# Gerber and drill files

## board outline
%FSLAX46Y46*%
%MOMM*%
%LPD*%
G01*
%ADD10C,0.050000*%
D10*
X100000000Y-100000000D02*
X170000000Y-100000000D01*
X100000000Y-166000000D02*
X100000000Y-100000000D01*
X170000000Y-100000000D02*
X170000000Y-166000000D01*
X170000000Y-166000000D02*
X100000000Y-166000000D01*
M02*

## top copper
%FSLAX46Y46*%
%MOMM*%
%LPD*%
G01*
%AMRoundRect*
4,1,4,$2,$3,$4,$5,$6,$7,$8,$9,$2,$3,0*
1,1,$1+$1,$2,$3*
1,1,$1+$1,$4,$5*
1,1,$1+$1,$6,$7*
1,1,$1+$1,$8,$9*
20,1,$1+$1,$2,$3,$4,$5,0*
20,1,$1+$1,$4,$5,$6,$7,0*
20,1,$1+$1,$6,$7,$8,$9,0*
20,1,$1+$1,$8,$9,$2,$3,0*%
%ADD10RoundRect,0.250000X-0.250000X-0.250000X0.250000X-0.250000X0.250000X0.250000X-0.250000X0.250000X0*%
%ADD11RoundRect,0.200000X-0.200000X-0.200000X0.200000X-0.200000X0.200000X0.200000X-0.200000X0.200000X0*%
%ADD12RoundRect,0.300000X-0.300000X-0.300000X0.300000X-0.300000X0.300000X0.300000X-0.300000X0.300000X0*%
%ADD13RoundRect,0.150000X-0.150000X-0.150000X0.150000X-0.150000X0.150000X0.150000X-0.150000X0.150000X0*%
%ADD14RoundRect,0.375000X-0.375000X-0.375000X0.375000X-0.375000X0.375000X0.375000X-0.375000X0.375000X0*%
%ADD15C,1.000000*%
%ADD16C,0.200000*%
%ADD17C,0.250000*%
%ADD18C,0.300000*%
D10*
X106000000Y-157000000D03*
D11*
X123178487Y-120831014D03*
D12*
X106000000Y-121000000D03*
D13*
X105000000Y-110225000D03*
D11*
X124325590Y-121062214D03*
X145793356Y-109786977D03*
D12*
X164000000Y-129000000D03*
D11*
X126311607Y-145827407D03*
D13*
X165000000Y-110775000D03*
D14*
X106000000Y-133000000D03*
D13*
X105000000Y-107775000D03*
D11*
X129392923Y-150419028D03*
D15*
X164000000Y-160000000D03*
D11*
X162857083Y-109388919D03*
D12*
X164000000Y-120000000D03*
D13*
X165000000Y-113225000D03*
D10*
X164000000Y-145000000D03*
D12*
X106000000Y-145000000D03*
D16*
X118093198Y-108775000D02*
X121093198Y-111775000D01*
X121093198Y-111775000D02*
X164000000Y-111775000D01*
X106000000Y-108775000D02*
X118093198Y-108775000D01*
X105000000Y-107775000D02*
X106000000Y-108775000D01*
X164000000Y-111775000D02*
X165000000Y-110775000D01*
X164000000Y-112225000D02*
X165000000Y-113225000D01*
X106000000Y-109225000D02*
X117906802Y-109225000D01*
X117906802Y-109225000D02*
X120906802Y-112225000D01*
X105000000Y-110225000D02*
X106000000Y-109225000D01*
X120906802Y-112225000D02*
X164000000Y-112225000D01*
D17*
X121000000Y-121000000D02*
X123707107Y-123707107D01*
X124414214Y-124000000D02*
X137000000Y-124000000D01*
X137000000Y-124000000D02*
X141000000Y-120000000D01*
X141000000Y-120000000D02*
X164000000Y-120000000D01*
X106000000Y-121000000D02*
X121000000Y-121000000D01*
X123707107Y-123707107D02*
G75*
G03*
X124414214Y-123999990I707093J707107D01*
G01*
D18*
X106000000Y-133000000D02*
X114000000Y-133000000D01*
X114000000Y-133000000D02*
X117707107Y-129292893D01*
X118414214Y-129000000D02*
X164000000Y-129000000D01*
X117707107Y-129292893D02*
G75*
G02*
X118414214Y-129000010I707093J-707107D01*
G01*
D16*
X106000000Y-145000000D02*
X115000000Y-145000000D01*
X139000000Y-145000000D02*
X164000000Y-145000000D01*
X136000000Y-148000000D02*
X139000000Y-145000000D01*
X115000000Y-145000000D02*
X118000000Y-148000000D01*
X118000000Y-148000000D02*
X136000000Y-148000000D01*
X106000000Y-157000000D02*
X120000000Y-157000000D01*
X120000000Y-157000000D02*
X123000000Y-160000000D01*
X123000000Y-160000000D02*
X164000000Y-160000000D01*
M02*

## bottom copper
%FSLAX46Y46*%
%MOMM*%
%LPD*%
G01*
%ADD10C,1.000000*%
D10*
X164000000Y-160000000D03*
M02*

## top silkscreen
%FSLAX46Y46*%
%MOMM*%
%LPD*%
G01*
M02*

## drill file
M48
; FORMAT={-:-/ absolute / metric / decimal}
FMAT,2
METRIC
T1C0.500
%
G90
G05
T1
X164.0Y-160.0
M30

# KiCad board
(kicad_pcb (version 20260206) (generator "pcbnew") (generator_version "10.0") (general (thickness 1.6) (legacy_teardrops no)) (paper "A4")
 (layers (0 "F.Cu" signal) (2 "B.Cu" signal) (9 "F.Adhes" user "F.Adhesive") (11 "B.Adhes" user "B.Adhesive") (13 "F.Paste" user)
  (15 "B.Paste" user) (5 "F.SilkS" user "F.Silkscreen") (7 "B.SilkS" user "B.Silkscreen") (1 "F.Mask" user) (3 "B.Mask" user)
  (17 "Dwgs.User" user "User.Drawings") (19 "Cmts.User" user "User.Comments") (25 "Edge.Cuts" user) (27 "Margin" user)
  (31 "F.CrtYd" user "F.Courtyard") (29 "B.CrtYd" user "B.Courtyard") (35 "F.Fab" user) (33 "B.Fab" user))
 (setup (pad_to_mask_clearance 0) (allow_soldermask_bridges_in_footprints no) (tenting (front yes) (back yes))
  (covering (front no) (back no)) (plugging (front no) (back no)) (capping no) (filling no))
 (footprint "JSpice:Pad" (layer "F.Cu") (at 106 157)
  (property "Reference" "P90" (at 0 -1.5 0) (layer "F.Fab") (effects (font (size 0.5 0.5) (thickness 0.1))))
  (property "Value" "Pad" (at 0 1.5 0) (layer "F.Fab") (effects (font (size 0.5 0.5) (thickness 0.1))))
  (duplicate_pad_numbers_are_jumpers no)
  (pad "1" smd roundrect (at 0 0) (size 1 1) (layers "F.Cu" "F.Mask") (roundrect_rratio 0.25) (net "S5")))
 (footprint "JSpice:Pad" (layer "F.Cu") (at 123.178487 120.831014)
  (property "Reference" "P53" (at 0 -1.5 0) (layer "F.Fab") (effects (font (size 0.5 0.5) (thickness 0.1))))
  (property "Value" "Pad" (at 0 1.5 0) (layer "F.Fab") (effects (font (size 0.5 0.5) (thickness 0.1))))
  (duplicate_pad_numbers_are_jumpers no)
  (pad "1" smd roundrect (at 0 0) (size 0.8 0.8) (layers "F.Cu" "F.Mask") (roundrect_rratio 0.25) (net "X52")))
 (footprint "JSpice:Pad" (layer "F.Cu") (at 106 121)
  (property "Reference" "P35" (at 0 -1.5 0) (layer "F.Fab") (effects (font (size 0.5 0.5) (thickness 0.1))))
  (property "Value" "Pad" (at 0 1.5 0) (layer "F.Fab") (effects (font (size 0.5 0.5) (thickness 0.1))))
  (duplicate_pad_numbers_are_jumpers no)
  (pad "1" smd roundrect (at 0 0) (size 1.2 1.2) (layers "F.Cu" "F.Mask") (roundrect_rratio 0.25) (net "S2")))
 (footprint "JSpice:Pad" (layer "F.Cu") (at 105 110.225)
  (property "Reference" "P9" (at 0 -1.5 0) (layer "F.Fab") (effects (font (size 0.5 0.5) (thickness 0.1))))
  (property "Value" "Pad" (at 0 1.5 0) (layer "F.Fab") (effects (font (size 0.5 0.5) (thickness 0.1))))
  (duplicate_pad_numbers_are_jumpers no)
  (pad "1" smd roundrect (at 0 0) (size 0.6 0.6) (layers "F.Cu" "F.Mask") (roundrect_rratio 0.25) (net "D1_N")))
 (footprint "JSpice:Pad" (layer "F.Cu") (at 124.32559 121.062214)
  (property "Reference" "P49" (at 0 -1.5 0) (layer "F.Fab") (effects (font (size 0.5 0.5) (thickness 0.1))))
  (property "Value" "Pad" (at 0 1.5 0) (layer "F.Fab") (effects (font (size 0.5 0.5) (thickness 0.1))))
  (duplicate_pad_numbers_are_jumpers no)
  (pad "1" smd roundrect (at 0 0) (size 0.8 0.8) (layers "F.Cu" "F.Mask") (roundrect_rratio 0.25) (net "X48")))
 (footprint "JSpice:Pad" (layer "F.Cu") (at 145.793356 109.786977)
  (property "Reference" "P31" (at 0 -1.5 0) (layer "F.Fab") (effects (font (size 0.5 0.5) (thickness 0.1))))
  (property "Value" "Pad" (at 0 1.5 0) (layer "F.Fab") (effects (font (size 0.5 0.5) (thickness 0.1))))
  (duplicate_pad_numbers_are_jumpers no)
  (pad "1" smd roundrect (at 0 0) (size 0.8 0.8) (layers "F.Cu" "F.Mask") (roundrect_rratio 0.25) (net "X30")))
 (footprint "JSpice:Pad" (layer "F.Cu") (at 164 129)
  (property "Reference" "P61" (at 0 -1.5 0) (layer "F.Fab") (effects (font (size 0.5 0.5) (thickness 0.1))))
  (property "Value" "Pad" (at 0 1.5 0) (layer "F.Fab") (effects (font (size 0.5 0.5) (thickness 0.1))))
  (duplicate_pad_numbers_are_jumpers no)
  (pad "1" smd roundrect (at 0 0) (size 1.2 1.2) (layers "F.Cu" "F.Mask") (roundrect_rratio 0.25) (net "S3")))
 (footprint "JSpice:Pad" (layer "F.Cu") (at 126.311607 145.827407)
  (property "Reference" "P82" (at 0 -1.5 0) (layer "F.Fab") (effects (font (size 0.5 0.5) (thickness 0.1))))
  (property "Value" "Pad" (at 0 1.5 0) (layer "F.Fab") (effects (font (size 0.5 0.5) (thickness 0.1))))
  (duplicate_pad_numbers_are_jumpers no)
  (pad "1" smd roundrect (at 0 0) (size 0.8 0.8) (layers "F.Cu" "F.Mask") (roundrect_rratio 0.25) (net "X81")))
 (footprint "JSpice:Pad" (layer "F.Cu") (at 165 110.775)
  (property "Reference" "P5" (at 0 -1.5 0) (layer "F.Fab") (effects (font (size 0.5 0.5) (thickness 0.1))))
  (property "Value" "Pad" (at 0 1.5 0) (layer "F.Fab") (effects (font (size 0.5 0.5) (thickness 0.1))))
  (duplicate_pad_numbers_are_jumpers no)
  (pad "1" smd roundrect (at 0 0) (size 0.6 0.6) (layers "F.Cu" "F.Mask") (roundrect_rratio 0.25) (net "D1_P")))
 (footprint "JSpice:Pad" (layer "F.Cu") (at 106 133)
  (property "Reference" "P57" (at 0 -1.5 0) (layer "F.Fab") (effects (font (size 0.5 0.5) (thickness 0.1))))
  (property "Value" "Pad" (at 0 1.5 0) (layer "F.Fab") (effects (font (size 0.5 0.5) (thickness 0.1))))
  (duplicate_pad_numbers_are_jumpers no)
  (pad "1" smd roundrect (at 0 0) (size 1.5 1.5) (layers "F.Cu" "F.Mask") (roundrect_rratio 0.25) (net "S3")))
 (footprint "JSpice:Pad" (layer "F.Cu") (at 105 107.775)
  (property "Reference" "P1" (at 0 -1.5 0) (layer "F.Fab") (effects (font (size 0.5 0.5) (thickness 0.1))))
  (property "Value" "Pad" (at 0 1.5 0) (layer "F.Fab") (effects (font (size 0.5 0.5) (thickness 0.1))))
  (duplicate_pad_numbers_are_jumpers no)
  (pad "1" smd roundrect (at 0 0) (size 0.6 0.6) (layers "F.Cu" "F.Mask") (roundrect_rratio 0.25) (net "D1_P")))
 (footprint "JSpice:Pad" (layer "F.Cu") (at 129.392923 150.419028)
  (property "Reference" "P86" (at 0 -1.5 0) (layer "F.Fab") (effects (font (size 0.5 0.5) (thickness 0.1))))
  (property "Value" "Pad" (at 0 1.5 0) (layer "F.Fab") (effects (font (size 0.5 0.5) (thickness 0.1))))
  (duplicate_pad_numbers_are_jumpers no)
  (pad "1" smd roundrect (at 0 0) (size 0.8 0.8) (layers "F.Cu" "F.Mask") (roundrect_rratio 0.25) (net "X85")))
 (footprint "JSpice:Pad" (layer "F.Cu") (at 164 160)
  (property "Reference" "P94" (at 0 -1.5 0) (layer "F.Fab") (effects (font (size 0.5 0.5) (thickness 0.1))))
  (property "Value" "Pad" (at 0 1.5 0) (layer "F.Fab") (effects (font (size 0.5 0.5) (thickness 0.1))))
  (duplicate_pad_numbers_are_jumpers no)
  (pad "1" thru_hole circle (at 0 0) (size 1 1) (drill 0.5) (layers "*.Cu" "*.Mask") (remove_unused_layers no) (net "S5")))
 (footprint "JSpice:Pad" (layer "F.Cu") (at 162.857083 109.388919)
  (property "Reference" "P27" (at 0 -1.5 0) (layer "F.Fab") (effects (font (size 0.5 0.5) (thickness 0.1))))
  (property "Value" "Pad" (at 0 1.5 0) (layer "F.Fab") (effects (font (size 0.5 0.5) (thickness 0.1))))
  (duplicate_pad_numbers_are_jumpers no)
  (pad "1" smd roundrect (at 0 0) (size 0.8 0.8) (layers "F.Cu" "F.Mask") (roundrect_rratio 0.25) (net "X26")))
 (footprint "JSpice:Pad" (layer "F.Cu") (at 164 120)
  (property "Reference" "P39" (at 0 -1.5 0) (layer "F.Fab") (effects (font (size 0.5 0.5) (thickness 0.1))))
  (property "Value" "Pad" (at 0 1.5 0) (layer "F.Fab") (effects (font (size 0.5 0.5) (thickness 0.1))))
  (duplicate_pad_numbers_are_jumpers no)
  (pad "1" smd roundrect (at 0 0) (size 1.2 1.2) (layers "F.Cu" "F.Mask") (roundrect_rratio 0.25) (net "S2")))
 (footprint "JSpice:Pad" (layer "F.Cu") (at 165 113.225)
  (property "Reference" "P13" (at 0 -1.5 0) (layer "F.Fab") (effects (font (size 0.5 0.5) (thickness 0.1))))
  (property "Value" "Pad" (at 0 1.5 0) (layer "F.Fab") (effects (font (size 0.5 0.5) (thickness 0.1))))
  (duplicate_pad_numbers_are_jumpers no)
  (pad "1" smd roundrect (at 0 0) (size 0.6 0.6) (layers "F.Cu" "F.Mask") (roundrect_rratio 0.25) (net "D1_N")))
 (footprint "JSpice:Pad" (layer "F.Cu") (at 164 145)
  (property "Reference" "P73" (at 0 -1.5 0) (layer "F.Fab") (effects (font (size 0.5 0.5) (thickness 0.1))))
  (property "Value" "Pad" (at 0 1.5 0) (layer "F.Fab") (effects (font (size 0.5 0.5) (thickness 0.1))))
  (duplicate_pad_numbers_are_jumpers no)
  (pad "1" smd roundrect (at 0 0) (size 1 1) (layers "F.Cu" "F.Mask") (roundrect_rratio 0.25) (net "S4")))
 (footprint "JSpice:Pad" (layer "F.Cu") (at 106 145)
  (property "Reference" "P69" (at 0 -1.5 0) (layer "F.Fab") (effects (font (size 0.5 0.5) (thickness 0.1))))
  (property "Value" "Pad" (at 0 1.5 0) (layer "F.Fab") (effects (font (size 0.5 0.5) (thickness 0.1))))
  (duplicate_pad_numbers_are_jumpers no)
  (pad "1" smd roundrect (at 0 0) (size 1.2 1.2) (layers "F.Cu" "F.Mask") (roundrect_rratio 0.25) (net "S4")))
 (gr_line (start 100 100) (end 170 100) (stroke (width 0.05) (type default)) (layer "Edge.Cuts"))
 (gr_line (start 100 166) (end 100 100) (stroke (width 0.05) (type default)) (layer "Edge.Cuts"))
 (gr_line (start 170 100) (end 170 166) (stroke (width 0.05) (type default)) (layer "Edge.Cuts"))
 (gr_line (start 170 166) (end 100 166) (stroke (width 0.05) (type default)) (layer "Edge.Cuts"))
 (segment (start 118.093198 108.775) (end 121.093198 111.775) (width 0.2) (layer "F.Cu") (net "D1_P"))
 (segment (start 121.093198 111.775) (end 164 111.775) (width 0.2) (layer "F.Cu") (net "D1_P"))
 (segment (start 106 108.775) (end 118.093198 108.775) (width 0.2) (layer "F.Cu") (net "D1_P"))
 (segment (start 105 107.775) (end 106 108.775) (width 0.2) (layer "F.Cu") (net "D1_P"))
 (segment (start 164 111.775) (end 165 110.775) (width 0.2) (layer "F.Cu") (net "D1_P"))
 (segment (start 164 112.225) (end 165 113.225) (width 0.2) (layer "F.Cu") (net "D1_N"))
 (segment (start 106 109.225) (end 117.906802 109.225) (width 0.2) (layer "F.Cu") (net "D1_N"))
 (segment (start 117.906802 109.225) (end 120.906802 112.225) (width 0.2) (layer "F.Cu") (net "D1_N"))
 (segment (start 105 110.225) (end 106 109.225) (width 0.2) (layer "F.Cu") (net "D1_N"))
 (segment (start 120.906802 112.225) (end 164 112.225) (width 0.2) (layer "F.Cu") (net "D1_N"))
 (segment (start 121 121) (end 123.707107 123.707107) (width 0.25) (layer "F.Cu") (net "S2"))
 (segment (start 124.414214 124) (end 137 124) (width 0.25) (layer "F.Cu") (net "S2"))
 (segment (start 137 124) (end 141 120) (width 0.25) (layer "F.Cu") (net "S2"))
 (segment (start 141 120) (end 164 120) (width 0.25) (layer "F.Cu") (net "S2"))
 (segment (start 106 121) (end 121 121) (width 0.25) (layer "F.Cu") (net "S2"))
 (arc (start 123.707107 123.707107) (mid 124.03153 123.92388) (end 124.414214 124) (width 0.25) (layer "F.Cu") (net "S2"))
 (segment (start 106 133) (end 114 133) (width 0.3) (layer "F.Cu") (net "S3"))
 (segment (start 114 133) (end 117.707107 129.292893) (width 0.3) (layer "F.Cu") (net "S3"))
 (segment (start 118.414214 129) (end 164 129) (width 0.3) (layer "F.Cu") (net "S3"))
 (arc (start 117.707107 129.292893) (mid 118.03153 129.07612) (end 118.414214 129) (width 0.3) (layer "F.Cu") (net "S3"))
 (segment (start 106 145) (end 115 145) (width 0.2) (layer "F.Cu") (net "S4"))
 (segment (start 139 145) (end 164 145) (width 0.2) (layer "F.Cu") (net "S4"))
 (segment (start 136 148) (end 139 145) (width 0.2) (layer "F.Cu") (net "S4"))
 (segment (start 115 145) (end 118 148) (width 0.2) (layer "F.Cu") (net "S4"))
 (segment (start 118 148) (end 136 148) (width 0.2) (layer "F.Cu") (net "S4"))
 (segment (start 106 157) (end 120 157) (width 0.2) (layer "F.Cu") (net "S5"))
 (segment (start 120 157) (end 123 160) (width 0.2) (layer "F.Cu") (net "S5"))
 (segment (start 123 160) (end 164 160) (width 0.2) (layer "F.Cu") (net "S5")))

